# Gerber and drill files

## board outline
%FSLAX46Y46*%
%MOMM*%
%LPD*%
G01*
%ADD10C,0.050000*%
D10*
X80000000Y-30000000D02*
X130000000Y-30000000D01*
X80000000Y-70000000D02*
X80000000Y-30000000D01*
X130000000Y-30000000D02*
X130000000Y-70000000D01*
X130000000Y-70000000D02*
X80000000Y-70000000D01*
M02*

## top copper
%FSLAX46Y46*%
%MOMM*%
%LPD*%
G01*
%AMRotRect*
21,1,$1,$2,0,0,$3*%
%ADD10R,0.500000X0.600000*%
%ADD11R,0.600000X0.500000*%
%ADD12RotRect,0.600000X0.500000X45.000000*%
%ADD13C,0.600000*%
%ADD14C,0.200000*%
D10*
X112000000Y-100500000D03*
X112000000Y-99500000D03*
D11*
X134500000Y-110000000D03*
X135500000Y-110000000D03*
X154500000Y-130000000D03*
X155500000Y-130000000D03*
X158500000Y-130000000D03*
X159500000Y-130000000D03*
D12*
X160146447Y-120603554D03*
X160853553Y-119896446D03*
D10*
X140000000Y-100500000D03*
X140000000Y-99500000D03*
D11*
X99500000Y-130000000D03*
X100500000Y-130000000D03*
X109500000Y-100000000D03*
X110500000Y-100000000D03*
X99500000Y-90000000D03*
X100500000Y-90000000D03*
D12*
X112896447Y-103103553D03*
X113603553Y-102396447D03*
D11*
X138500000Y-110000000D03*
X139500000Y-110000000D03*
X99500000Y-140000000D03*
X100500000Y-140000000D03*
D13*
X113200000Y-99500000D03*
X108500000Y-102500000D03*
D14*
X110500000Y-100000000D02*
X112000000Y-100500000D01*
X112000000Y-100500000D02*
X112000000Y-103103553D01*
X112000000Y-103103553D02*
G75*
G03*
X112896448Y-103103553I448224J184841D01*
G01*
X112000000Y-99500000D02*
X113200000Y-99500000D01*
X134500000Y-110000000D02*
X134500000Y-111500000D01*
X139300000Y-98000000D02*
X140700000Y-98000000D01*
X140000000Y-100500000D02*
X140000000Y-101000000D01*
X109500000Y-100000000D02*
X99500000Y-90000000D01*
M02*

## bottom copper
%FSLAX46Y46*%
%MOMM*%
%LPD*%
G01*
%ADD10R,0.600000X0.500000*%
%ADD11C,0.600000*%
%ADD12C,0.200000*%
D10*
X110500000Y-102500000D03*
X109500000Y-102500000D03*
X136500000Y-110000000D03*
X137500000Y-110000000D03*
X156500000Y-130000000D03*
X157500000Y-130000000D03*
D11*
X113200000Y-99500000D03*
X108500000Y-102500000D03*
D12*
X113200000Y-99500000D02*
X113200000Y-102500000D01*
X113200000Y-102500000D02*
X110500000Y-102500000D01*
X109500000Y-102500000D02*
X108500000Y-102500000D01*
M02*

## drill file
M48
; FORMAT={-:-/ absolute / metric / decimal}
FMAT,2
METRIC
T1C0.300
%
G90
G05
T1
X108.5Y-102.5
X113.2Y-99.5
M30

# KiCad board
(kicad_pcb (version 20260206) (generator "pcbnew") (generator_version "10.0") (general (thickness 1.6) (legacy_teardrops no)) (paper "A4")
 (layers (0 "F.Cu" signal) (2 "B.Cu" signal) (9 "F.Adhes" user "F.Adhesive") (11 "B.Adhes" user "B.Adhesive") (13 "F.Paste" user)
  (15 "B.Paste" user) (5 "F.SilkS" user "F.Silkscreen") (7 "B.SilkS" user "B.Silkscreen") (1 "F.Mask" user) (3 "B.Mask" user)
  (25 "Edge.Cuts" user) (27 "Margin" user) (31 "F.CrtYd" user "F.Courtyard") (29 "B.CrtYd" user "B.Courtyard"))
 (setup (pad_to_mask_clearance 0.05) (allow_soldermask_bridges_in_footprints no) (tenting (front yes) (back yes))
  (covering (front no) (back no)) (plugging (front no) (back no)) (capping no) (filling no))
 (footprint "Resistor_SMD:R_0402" (layer "F.Cu") (at 112 100 90)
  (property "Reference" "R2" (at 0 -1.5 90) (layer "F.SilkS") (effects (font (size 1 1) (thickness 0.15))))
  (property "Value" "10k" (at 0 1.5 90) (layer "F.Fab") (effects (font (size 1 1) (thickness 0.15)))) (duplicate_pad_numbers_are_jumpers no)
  (pad "1" smd rect (at -0.5 0 90) (size 0.6 0.5) (layers "F.Cu" "F.Mask" "F.Paste") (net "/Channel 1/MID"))
  (pad "2" smd rect (at 0.5 0 90) (size 0.6 0.5) (layers "F.Cu" "F.Mask" "F.Paste") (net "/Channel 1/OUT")))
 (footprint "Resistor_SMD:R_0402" (layer "F.Cu") (at 135 110)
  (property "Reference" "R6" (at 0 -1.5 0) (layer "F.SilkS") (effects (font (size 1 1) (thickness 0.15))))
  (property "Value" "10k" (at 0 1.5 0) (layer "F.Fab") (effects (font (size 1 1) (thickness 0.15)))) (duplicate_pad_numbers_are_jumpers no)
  (pad "1" smd rect (at -0.5 0) (size 0.6 0.5) (layers "F.Cu" "F.Mask" "F.Paste") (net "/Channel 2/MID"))
  (pad "2" smd rect (at 0.5 0) (size 0.6 0.5) (layers "F.Cu" "F.Mask" "F.Paste") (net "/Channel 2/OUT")))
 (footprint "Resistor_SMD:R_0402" (layer "F.Cu") (at 155 130)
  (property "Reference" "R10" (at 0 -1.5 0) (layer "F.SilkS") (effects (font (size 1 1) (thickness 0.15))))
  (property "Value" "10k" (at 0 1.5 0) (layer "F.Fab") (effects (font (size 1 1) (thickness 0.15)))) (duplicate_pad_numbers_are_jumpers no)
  (pad "1" smd rect (at -0.5 0) (size 0.6 0.5) (layers "F.Cu" "F.Mask" "F.Paste") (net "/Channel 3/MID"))
  (pad "2" smd rect (at 0.5 0) (size 0.6 0.5) (layers "F.Cu" "F.Mask" "F.Paste") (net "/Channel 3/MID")))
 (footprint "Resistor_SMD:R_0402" (layer "F.Cu") (at 159 130)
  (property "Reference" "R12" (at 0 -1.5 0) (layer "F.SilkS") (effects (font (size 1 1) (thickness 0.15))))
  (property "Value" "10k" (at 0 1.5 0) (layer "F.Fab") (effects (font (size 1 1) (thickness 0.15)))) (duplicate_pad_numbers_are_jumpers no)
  (pad "1" smd rect (at -0.5 0) (size 0.6 0.5) (layers "F.Cu" "F.Mask" "F.Paste") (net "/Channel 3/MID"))
  (pad "2" smd rect (at 0.5 0) (size 0.6 0.5) (layers "F.Cu" "F.Mask" "F.Paste") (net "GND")))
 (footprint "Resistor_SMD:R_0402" (layer "F.Cu") (at 160.5 120.25 45)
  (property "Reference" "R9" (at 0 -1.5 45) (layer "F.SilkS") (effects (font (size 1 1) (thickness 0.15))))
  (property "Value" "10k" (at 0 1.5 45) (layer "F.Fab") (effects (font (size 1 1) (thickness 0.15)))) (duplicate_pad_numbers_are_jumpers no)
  (pad "1" smd rect (at -0.5 0.000001 45) (size 0.6 0.5) (layers "F.Cu" "F.Mask" "F.Paste") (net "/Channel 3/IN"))
  (pad "2" smd rect (at 0.5 -0.000001 45) (size 0.6 0.5) (layers "F.Cu" "F.Mask" "F.Paste") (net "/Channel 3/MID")))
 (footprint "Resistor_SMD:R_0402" (layer "F.Cu") (at 140 100 90)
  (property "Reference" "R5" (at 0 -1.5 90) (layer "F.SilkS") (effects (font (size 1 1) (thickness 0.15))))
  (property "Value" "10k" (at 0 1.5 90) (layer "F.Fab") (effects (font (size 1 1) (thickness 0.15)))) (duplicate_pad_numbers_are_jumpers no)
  (pad "1" smd rect (at -0.5 0 90) (size 0.6 0.5) (layers "F.Cu" "F.Mask" "F.Paste") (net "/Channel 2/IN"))
  (pad "2" smd rect (at 0.5 0 90) (size 0.6 0.5) (layers "F.Cu" "F.Mask" "F.Paste") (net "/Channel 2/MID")))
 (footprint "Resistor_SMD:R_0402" (layer "F.Cu") (at 100 130)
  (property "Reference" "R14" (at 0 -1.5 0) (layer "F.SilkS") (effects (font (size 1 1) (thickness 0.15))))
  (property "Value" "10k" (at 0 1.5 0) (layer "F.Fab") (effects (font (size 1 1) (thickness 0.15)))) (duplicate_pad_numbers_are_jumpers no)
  (pad "1" smd rect (at -0.5 0) (size 0.6 0.5) (layers "F.Cu" "F.Mask" "F.Paste") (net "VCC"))
  (pad "2" smd rect (at 0.5 0) (size 0.6 0.5) (layers "F.Cu" "F.Mask" "F.Paste") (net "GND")))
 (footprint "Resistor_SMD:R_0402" (layer "F.Cu") (at 110 100)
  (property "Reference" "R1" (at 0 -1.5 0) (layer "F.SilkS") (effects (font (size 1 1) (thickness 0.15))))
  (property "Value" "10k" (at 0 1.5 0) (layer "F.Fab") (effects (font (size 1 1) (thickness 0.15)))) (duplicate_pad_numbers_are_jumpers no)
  (pad "1" smd rect (at -0.5 0) (size 0.6 0.5) (layers "F.Cu" "F.Mask" "F.Paste") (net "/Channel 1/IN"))
  (pad "2" smd rect (at 0.5 0) (size 0.6 0.5) (layers "F.Cu" "F.Mask" "F.Paste") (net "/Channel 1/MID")))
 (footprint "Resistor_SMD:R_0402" (layer "F.Cu") (at 100 90)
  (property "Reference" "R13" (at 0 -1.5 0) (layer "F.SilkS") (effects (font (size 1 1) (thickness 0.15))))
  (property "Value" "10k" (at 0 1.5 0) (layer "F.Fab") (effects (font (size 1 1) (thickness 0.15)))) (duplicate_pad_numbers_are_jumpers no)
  (pad "1" smd rect (at -0.5 0) (size 0.6 0.5) (layers "F.Cu" "F.Mask" "F.Paste") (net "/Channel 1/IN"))
  (pad "2" smd rect (at 0.5 0) (size 0.6 0.5) (layers "F.Cu" "F.Mask" "F.Paste") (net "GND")))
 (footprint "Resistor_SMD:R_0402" (layer "F.Cu") (at 113.25 102.75 45)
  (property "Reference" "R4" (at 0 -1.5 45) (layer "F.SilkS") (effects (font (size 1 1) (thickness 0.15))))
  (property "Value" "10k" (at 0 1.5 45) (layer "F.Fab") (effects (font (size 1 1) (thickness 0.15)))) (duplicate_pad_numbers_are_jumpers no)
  (pad "1" smd rect (at -0.499999 0 45) (size 0.6 0.5) (layers "F.Cu" "F.Mask" "F.Paste") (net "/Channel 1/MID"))
  (pad "2" smd rect (at 0.499999 0 45) (size 0.6 0.5) (layers "F.Cu" "F.Mask" "F.Paste") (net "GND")))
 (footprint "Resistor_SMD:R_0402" (layer "F.Cu") (at 139 110)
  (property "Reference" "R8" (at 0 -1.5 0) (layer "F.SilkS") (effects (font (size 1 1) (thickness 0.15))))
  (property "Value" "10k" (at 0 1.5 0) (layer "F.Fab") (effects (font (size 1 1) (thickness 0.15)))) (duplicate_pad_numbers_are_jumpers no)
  (pad "1" smd rect (at -0.5 0) (size 0.6 0.5) (layers "F.Cu" "F.Mask" "F.Paste") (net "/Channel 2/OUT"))
  (pad "2" smd rect (at 0.5 0) (size 0.6 0.5) (layers "F.Cu" "F.Mask" "F.Paste") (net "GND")))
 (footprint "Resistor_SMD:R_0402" (layer "F.Cu") (at 100 140)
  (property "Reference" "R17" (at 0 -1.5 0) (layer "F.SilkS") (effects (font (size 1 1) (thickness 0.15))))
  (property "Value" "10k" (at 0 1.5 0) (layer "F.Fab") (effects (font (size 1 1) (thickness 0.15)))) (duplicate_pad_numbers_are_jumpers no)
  (pad "1" smd rect (at -0.5 0) (size 0.6 0.5) (layers "F.Cu" "F.Mask" "F.Paste") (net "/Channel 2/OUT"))
  (pad "2" smd rect (at 0.5 0) (size 0.6 0.5) (layers "F.Cu" "F.Mask" "F.Paste") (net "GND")))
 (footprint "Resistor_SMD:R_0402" (layer "B.Cu") (at 110 102.5 180)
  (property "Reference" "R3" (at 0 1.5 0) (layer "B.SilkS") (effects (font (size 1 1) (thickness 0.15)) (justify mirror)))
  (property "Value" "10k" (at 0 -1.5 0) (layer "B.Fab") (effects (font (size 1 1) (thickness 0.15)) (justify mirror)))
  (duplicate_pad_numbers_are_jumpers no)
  (pad "1" smd rect (at -0.5 0 180) (size 0.6 0.5) (layers "B.Cu" "B.Mask" "B.Paste") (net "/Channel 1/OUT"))
  (pad "2" smd rect (at 0.5 0 180) (size 0.6 0.5) (layers "B.Cu" "B.Mask" "B.Paste") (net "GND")))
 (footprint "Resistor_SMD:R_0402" (layer "B.Cu") (at 137 110)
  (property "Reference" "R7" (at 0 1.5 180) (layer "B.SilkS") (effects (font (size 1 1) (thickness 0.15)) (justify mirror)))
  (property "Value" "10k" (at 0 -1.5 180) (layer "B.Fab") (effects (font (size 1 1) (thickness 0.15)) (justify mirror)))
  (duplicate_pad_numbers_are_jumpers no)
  (pad "1" smd rect (at -0.5 0) (size 0.6 0.5) (layers "B.Cu" "B.Mask" "B.Paste") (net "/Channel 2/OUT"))
  (pad "2" smd rect (at 0.5 0) (size 0.6 0.5) (layers "B.Cu" "B.Mask" "B.Paste") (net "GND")))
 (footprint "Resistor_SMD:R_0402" (layer "B.Cu") (at 157 130)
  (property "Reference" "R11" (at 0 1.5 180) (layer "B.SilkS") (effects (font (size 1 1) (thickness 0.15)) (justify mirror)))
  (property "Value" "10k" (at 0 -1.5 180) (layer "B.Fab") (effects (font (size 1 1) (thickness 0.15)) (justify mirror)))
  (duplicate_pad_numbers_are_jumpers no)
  (pad "1" smd rect (at -0.5 0) (size 0.6 0.5) (layers "B.Cu" "B.Mask" "B.Paste") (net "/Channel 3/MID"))
  (pad "2" smd rect (at 0.5 0) (size 0.6 0.5) (layers "B.Cu" "B.Mask" "B.Paste") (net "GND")))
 (gr_line (start 80 30) (end 130 30) (stroke (width 0.05) (type default)) (layer "Edge.Cuts"))
 (gr_line (start 80 70) (end 80 30) (stroke (width 0.05) (type default)) (layer "Edge.Cuts"))
 (gr_line (start 130 30) (end 130 70) (stroke (width 0.05) (type default)) (layer "Edge.Cuts"))
 (gr_line (start 130 70) (end 80 70) (stroke (width 0.05) (type default)) (layer "Edge.Cuts"))
 (segment (start 110.5 100) (end 112 100.5) (width 0.2) (locked yes) (layer "F.Cu") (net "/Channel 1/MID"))
 (segment (start 112 100.5) (end 112 103.103553) (width 0.2) (layer "F.Cu") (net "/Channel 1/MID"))
 (arc (start 112 103.103553) (mid 112.448223 103.403553) (end 112.896447 103.103553) (width 0.2) (layer "F.Cu") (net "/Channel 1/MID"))
 (segment (start 112 99.5) (end 113.2 99.5) (width 0.2) (layer "F.Cu") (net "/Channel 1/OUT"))
 (via (at 113.2 99.5) (size 0.6) (drill 0.3) (layers "F.Cu" "B.Cu") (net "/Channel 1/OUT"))
 (segment (start 113.2 99.5) (end 113.2 102.5) (width 0.2) (layer "B.Cu") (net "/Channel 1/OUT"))
 (segment (start 113.2 102.5) (end 110.5 102.5) (width 0.2) (layer "B.Cu") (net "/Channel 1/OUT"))
 (segment (start 134.5 110) (end 134.5 111.5) (width 0.2) (layer "F.Cu") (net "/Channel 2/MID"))
 (segment (start 139.3 98) (end 140.7 98) (width 0.2) (layer "F.Cu") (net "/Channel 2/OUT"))
 (via (at 108.5 102.5) (size 0.6) (drill 0.3) (layers "F.Cu" "B.Cu") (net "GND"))
 (segment (start 109.5 102.5) (end 108.5 102.5) (width 0.2) (layer "B.Cu") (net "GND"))
 (segment (start 140 100.5) (end 140 101) (width 0.2) (layer "F.Cu") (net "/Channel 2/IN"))
 (segment (start 109.5 100) (end 99.5 90) (width 0.2) (layer "F.Cu") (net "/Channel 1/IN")))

